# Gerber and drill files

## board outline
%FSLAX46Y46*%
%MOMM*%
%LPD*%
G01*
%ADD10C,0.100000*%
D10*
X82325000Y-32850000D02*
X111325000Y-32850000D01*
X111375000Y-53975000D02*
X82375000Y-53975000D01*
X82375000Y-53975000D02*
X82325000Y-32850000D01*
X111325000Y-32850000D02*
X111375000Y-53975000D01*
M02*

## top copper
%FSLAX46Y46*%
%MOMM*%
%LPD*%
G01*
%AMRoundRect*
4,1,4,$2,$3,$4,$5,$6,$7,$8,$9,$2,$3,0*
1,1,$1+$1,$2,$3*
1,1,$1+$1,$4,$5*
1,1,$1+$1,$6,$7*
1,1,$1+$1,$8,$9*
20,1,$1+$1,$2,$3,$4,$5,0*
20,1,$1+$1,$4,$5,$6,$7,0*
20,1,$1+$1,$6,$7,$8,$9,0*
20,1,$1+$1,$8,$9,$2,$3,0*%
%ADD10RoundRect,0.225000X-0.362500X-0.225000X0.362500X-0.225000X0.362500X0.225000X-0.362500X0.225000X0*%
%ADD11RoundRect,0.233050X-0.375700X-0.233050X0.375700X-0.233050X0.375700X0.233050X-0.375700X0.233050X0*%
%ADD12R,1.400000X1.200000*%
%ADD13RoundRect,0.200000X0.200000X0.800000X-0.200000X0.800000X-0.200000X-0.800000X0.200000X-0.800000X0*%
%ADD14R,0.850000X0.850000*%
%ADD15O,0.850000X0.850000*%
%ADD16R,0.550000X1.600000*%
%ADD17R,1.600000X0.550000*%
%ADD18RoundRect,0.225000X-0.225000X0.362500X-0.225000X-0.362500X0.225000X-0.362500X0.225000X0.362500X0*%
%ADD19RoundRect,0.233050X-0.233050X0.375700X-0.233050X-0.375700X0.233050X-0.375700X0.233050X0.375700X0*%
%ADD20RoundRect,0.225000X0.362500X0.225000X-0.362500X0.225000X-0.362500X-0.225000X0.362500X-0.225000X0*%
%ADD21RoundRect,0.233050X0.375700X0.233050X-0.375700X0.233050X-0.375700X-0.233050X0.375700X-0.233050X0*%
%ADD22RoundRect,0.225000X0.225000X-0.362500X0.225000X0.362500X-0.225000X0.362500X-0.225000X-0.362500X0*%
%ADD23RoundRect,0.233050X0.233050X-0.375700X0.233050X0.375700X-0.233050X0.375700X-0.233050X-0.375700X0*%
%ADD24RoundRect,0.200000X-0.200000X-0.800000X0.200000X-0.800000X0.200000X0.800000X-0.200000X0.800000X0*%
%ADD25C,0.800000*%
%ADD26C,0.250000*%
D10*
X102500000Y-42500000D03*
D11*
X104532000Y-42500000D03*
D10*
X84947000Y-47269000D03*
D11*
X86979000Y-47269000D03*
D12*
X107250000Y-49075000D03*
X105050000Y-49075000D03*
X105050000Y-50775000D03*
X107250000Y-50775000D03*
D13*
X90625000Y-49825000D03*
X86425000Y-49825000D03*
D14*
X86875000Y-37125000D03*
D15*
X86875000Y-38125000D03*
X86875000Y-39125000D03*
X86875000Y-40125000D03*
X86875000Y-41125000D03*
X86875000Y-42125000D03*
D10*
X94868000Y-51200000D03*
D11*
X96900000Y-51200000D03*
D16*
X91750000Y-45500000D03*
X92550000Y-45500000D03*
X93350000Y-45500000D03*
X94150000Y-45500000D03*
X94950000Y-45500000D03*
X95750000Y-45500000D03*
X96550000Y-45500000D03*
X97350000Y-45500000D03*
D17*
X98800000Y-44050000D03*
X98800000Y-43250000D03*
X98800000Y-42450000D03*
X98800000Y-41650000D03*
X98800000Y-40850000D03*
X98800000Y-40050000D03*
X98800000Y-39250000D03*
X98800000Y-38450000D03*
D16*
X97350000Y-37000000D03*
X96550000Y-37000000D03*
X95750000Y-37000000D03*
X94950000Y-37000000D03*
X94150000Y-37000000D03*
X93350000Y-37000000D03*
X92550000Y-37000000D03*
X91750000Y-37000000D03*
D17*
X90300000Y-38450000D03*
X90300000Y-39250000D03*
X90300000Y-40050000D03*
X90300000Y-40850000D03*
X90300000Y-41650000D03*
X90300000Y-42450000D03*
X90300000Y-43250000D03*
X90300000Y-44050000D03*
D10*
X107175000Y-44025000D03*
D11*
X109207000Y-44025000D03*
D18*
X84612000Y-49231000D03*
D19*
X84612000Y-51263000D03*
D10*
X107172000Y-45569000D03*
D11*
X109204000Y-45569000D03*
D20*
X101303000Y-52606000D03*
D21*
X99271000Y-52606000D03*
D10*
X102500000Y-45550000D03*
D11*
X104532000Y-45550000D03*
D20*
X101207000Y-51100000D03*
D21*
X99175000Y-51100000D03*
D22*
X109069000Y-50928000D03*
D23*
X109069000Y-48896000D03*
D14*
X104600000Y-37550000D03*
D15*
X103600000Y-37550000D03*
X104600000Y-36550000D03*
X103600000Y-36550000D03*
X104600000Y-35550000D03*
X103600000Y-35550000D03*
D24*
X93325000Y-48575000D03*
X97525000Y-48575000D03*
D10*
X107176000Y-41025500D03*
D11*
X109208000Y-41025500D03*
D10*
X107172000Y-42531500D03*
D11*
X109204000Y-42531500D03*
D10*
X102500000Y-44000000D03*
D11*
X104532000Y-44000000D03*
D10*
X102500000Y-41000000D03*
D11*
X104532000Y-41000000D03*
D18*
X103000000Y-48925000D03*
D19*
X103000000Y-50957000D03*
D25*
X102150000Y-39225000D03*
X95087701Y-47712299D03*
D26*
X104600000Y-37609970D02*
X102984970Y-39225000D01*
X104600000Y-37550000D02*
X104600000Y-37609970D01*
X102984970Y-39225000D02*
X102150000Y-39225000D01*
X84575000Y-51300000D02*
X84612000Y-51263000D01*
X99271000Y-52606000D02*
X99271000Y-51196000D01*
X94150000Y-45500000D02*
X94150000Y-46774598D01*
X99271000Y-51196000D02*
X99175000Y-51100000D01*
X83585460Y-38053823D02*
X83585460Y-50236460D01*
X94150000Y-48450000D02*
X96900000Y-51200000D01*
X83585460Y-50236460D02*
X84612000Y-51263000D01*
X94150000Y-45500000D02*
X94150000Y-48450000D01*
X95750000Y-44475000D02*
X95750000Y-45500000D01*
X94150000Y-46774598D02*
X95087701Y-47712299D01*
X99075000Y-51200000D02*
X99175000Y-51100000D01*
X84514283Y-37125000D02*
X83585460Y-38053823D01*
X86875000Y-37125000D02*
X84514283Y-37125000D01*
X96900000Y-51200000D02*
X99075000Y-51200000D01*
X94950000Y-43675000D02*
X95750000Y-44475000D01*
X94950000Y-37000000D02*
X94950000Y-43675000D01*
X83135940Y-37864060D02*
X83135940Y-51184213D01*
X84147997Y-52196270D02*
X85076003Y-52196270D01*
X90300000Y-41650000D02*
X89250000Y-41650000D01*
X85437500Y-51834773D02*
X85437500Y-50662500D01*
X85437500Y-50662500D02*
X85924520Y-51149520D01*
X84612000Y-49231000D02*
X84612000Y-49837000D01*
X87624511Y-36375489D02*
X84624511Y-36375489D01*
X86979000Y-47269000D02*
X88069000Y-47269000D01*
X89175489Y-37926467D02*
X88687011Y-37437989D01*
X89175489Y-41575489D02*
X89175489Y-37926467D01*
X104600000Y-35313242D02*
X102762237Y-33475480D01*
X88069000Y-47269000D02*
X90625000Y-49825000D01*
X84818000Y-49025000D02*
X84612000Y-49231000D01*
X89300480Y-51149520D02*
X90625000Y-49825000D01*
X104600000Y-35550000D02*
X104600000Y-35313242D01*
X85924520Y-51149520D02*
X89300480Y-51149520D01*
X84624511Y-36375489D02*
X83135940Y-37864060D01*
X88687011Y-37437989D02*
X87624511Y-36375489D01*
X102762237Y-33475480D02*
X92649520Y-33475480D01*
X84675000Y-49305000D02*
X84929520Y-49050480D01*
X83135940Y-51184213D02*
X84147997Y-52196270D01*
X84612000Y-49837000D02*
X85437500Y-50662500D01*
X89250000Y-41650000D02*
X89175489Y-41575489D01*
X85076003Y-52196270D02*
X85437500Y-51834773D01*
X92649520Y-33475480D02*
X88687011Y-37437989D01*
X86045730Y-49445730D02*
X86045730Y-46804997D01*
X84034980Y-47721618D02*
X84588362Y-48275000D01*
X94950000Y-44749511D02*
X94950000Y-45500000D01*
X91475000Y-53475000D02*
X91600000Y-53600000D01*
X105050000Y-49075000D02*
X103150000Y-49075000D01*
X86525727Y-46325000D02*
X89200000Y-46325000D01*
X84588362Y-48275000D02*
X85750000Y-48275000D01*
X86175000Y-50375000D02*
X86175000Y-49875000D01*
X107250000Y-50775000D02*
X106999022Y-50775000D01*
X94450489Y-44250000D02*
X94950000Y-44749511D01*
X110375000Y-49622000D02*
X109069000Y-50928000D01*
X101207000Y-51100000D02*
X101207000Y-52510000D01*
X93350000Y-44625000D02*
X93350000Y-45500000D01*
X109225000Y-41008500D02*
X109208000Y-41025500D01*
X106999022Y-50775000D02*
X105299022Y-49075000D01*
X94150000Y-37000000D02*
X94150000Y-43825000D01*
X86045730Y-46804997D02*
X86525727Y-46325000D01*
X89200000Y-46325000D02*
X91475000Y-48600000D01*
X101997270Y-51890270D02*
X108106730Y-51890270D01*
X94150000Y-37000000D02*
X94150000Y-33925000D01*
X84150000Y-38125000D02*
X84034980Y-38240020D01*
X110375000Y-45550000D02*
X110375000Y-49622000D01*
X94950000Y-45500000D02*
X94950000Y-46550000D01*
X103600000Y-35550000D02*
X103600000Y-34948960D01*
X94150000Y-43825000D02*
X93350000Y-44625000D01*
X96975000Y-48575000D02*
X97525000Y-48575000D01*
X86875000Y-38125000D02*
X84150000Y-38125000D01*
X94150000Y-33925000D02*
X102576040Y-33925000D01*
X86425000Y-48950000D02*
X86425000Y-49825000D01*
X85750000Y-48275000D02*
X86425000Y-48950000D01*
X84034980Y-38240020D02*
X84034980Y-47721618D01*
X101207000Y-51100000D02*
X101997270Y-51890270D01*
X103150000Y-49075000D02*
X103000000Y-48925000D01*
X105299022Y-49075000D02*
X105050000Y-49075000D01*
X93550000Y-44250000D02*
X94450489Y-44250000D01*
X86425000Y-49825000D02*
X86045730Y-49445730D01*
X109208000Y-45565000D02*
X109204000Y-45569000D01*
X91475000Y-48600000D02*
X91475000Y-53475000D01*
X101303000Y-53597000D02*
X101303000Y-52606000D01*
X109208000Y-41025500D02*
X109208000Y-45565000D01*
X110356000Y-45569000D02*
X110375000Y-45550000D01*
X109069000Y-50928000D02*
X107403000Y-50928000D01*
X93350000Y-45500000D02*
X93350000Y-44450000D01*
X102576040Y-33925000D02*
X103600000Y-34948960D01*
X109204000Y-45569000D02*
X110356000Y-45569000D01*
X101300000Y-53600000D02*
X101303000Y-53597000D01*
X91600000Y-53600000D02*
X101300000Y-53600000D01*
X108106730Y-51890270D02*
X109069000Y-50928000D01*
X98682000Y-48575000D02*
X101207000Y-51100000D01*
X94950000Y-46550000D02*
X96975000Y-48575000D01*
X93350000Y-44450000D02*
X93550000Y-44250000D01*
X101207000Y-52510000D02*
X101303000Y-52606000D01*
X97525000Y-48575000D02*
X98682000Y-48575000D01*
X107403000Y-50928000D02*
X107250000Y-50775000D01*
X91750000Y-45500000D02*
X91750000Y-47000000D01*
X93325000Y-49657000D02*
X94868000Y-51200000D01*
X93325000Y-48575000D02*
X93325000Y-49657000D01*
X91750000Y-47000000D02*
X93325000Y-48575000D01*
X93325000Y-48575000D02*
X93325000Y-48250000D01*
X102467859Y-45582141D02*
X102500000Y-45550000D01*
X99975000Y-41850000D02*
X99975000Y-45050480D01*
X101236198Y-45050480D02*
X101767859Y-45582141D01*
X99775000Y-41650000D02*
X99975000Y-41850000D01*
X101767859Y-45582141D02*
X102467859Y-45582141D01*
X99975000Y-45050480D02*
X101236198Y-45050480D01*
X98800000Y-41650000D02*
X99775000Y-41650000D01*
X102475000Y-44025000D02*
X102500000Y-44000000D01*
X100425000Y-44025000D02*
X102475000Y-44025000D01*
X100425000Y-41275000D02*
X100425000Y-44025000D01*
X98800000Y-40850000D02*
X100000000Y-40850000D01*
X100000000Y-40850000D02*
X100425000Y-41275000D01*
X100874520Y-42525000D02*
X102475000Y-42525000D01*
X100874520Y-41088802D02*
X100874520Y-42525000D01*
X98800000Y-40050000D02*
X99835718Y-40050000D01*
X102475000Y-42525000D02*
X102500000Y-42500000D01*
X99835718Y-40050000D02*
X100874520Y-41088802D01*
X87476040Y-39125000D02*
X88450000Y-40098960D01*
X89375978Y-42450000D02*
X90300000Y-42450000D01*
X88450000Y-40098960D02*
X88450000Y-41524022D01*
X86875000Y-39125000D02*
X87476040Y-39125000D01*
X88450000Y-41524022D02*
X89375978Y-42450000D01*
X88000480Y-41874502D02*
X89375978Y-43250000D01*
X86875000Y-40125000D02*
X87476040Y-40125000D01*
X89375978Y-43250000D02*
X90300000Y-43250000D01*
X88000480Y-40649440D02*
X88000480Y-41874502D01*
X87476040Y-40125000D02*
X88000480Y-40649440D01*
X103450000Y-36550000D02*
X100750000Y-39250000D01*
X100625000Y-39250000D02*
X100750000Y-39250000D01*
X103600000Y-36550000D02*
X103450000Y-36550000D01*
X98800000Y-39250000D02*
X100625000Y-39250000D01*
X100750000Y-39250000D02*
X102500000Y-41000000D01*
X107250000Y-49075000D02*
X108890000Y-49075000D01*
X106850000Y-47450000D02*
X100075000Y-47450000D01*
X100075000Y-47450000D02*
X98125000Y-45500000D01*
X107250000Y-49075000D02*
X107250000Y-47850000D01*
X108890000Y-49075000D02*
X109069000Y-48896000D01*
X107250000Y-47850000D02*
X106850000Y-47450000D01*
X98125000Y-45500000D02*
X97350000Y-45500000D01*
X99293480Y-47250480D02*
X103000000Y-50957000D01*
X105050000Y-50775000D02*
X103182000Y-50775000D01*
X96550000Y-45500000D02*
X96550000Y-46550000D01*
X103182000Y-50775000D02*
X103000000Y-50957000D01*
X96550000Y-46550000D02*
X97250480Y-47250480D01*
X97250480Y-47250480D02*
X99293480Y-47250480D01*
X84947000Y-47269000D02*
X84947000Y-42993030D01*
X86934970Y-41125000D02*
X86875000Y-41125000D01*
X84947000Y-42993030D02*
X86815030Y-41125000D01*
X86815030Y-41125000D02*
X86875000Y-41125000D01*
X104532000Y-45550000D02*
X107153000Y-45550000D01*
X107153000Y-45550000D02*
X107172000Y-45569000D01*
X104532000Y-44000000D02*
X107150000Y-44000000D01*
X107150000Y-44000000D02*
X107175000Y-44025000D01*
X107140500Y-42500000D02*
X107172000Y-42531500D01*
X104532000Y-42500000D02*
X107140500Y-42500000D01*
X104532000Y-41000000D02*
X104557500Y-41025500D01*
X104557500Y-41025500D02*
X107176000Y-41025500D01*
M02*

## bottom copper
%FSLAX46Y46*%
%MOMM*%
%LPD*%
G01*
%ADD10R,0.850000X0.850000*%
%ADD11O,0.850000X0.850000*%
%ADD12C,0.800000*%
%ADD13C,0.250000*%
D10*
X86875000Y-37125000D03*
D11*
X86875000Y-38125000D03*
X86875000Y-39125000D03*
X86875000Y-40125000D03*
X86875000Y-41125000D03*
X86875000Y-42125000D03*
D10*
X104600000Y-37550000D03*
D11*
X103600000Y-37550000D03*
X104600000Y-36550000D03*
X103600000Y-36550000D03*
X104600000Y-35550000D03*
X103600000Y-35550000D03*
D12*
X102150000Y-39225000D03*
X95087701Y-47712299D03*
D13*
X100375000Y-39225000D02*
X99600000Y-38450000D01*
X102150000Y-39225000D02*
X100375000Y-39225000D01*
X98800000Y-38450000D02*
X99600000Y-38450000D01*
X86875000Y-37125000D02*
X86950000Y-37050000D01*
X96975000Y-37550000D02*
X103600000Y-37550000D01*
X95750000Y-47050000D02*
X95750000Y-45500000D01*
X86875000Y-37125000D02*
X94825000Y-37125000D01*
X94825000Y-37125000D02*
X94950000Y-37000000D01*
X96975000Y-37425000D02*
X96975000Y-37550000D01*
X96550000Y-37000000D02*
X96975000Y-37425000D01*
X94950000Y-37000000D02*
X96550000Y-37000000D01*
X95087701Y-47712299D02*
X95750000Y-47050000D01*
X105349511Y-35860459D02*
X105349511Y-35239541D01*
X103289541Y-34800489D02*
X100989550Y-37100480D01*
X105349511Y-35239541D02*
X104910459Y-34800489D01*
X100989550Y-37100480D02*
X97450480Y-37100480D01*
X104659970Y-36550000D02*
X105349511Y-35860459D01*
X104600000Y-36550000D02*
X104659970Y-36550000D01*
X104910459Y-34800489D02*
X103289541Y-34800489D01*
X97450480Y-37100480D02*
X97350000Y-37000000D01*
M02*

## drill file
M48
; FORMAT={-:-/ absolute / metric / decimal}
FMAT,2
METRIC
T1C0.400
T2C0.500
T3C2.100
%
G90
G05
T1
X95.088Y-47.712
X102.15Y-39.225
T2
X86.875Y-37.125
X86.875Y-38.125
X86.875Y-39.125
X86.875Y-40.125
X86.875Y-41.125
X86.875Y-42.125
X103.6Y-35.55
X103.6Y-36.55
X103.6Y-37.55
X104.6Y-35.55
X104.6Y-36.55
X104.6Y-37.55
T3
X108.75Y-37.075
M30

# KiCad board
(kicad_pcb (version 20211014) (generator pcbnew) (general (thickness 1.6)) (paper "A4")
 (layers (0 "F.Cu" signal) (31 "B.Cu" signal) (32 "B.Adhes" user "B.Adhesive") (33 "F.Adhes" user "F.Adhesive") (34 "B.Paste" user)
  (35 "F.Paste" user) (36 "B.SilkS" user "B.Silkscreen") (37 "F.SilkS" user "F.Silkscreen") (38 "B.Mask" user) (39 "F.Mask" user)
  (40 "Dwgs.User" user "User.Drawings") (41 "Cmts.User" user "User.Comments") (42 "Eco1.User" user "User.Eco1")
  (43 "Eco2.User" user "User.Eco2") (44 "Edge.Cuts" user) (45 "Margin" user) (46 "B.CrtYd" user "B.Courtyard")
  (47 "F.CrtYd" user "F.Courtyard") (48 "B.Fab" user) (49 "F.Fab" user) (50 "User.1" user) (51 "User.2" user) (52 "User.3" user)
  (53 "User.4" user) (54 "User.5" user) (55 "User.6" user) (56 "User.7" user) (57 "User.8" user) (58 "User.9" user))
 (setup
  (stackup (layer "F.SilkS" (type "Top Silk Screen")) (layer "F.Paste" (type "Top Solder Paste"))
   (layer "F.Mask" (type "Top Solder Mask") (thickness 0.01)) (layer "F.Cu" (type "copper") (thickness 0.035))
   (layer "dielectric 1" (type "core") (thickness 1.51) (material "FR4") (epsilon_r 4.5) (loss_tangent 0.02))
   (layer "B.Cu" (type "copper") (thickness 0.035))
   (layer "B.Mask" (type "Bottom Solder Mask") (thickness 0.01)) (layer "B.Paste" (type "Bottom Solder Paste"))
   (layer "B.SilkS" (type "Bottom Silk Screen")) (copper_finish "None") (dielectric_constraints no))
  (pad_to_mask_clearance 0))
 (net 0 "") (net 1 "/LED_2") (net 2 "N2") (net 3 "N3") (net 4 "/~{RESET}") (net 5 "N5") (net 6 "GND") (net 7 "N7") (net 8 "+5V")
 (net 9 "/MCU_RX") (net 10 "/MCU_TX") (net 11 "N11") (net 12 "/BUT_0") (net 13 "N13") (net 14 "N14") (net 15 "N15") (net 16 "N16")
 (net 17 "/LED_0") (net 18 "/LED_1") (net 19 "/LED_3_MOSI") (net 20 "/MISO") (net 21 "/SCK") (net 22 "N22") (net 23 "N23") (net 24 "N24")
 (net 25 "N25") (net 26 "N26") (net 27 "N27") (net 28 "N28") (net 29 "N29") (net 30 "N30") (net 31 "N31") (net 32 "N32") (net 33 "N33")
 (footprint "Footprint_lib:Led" (layer "F.Cu") (at 103.478 42.481)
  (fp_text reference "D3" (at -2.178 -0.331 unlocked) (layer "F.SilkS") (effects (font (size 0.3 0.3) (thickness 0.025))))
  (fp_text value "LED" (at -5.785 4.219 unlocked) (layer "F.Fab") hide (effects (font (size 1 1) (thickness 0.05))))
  (pad "1" smd roundrect (at -0.978 0.019) (size 1.175 0.9) (layers "F.Cu" "F.Paste" "F.Mask") (roundrect_rratio 0.25) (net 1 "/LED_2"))
  (pad "2" smd roundrect (at 1.054 0.019) (size 1.2175 0.9322) (layers "F.Cu" "F.Paste" "F.Mask") (roundrect_rratio 0.25) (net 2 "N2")))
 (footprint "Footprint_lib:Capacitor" (layer "F.Cu") (at 85.95 47.25)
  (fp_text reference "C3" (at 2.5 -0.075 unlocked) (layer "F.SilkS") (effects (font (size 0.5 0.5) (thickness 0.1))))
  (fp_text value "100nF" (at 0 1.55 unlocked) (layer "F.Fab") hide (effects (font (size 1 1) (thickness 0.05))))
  (pad "1" smd roundrect (at -1.003 0.019) (size 1.175 0.9) (layers "F.Cu" "F.Paste" "F.Mask") (roundrect_rratio 0.25) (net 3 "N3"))
  (pad "2" smd roundrect (at 1.029 0.019) (size 1.2175 0.9322) (layers "F.Cu" "F.Paste" "F.Mask") (roundrect_rratio 0.25)
   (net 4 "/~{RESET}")))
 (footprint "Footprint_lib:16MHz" (layer "F.Cu") (at 106.15 49.875 180)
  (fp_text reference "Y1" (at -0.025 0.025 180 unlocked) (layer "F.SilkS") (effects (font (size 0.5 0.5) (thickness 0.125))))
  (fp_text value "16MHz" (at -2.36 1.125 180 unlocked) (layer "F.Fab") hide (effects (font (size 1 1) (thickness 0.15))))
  (pad "1" smd rect (at -1.1 0.8 180) (size 1.4 1.2) (layers "F.Cu" "F.Paste" "F.Mask") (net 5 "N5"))
  (pad "2" smd rect (at 1.1 0.8 180) (size 1.4 1.2) (layers "F.Cu" "F.Paste" "F.Mask") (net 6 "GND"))
  (pad "3" smd rect (at 1.1 -0.9 180) (size 1.4 1.2) (layers "F.Cu" "F.Paste" "F.Mask") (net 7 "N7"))
  (pad "4" smd rect (at -1.1 -0.9 180) (size 1.4 1.2) (layers "F.Cu" "F.Paste" "F.Mask") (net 6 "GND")))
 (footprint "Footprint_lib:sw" (layer "F.Cu") (at 88.525 49.895 180)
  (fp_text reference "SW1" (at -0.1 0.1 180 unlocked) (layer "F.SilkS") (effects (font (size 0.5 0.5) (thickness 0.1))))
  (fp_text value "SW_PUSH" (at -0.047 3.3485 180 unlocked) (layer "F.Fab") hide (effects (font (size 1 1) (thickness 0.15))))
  (pad "1" smd roundrect (at -2.1 0.07 180) (size 0.8 2) (layers "F.Cu" "F.Paste" "F.Mask") (roundrect_rratio 0.25) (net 4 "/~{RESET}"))
  (pad "2" smd roundrect (at 2.1 0.07 180) (size 0.8 2) (layers "F.Cu" "F.Paste" "F.Mask") (roundrect_rratio 0.25) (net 6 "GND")))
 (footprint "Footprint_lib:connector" (layer "F.Cu") (at 86.875 39.625)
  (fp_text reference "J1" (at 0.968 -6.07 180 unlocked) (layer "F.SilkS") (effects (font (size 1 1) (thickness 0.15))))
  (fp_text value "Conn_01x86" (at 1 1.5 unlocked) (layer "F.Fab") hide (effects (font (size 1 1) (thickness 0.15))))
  (pad "1" thru_hole rect (at 0 -2.5) (size 0.85 0.85) (drill 0.5) (layers *.Cu *.Mask) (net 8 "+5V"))
  (pad "2" thru_hole oval (at 0 -1.5) (size 0.85 0.85) (drill 0.5) (layers *.Cu *.Mask) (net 6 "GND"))
  (pad "3" thru_hole oval (at 0 -0.5) (size 0.85 0.85) (drill 0.5) (layers *.Cu *.Mask) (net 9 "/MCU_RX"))
  (pad "4" thru_hole oval (at 0 0.5) (size 0.85 0.85) (drill 0.5) (layers *.Cu *.Mask) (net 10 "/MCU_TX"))
  (pad "5" thru_hole oval (at 0 1.5) (size 0.85 0.85) (drill 0.5) (layers *.Cu *.Mask) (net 3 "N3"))
  (pad "6" thru_hole oval (at 0 2.5) (size 0.85 0.85) (drill 0.5) (layers *.Cu *.Mask) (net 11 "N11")))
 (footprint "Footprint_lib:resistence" (layer "F.Cu") (at 95.921 51.1685)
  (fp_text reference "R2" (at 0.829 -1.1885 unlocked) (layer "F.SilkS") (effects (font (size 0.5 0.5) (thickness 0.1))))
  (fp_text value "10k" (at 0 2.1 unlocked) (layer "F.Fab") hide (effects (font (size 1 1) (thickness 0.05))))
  (pad "1" smd roundrect (at -1.053 0.0315) (size 1.175 0.9) (layers "F.Cu" "F.Paste" "F.Mask") (roundrect_rratio 0.25) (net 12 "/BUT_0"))
  (pad "2" smd roundrect (at 0.979 0.0315) (size 1.2175 0.9322) (layers "F.Cu" "F.Paste" "F.Mask") (roundrect_rratio 0.25) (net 8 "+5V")))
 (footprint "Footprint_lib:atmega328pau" (layer "F.Cu") (at 94.55 41.25 90)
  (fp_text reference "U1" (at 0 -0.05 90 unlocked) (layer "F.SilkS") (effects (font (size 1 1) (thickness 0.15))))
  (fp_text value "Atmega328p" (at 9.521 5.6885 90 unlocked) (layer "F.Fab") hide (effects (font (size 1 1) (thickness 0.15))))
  (pad "1" smd rect (at -4.25 -2.8 90) (size 1.6 0.55) (layers "F.Cu" "F.Paste" "F.Mask") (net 12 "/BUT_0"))
  (pad "2" smd rect (at -4.25 -2 90) (size 1.6 0.55) (layers "F.Cu" "F.Paste" "F.Mask") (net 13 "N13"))
  (pad "3" smd rect (at -4.25 -1.2 90) (size 1.6 0.55) (layers "F.Cu" "F.Paste" "F.Mask") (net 6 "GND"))
  (pad "4" smd rect (at -4.25 -0.4 90) (size 1.6 0.55) (layers "F.Cu" "F.Paste" "F.Mask") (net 8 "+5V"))
  (pad "5" smd rect (at -4.25 0.4 90) (size 1.6 0.55) (layers "F.Cu" "F.Paste" "F.Mask") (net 6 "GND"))
  (pad "6" smd rect (at -4.25 1.2 90) (size 1.6 0.55) (layers "F.Cu" "F.Paste" "F.Mask") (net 8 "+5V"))
  (pad "7" smd rect (at -4.25 2 90) (size 1.6 0.55) (layers "F.Cu" "F.Paste" "F.Mask") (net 7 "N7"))
  (pad "8" smd rect (at -4.25 2.8 90) (size 1.6 0.55) (layers "F.Cu" "F.Paste" "F.Mask") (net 5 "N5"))
  (pad "9" smd rect (at -2.8 4.25 180) (size 1.6 0.55) (layers "F.Cu" "F.Paste" "F.Mask") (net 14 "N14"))
  (pad "10" smd rect (at -2 4.25 180) (size 1.6 0.55) (layers "F.Cu" "F.Paste" "F.Mask") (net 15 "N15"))
  (pad "11" smd rect (at -1.2 4.25 180) (size 1.6 0.55) (layers "F.Cu" "F.Paste" "F.Mask") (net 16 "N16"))
  (pad "12" smd rect (at -0.4 4.25 180) (size 1.6 0.55) (layers "F.Cu" "F.Paste" "F.Mask") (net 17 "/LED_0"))
  (pad "13" smd rect (at 0.4 4.25 180) (size 1.6 0.55) (layers "F.Cu" "F.Paste" "F.Mask") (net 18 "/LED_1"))
  (pad "14" smd rect (at 1.2 4.25 180) (size 1.6 0.55) (layers "F.Cu" "F.Paste" "F.Mask") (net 1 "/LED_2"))
  (pad "15" smd rect (at 2 4.25 180) (size 1.6 0.55) (layers "F.Cu" "F.Paste" "F.Mask") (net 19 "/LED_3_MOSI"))
  (pad "16" smd rect (at 2.8 4.25 180) (size 1.6 0.55) (layers "F.Cu" "F.Paste" "F.Mask") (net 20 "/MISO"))
  (pad "17" smd rect (at 4.25 2.8 90) (size 1.6 0.55) (layers "F.Cu" "F.Paste" "F.Mask") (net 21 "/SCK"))
  (pad "18" smd rect (at 4.25 2 90) (size 1.6 0.55) (layers "F.Cu" "F.Paste" "F.Mask") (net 8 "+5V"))
  (pad "19" smd rect (at 4.25 1.2 90) (size 1.6 0.55) (layers "F.Cu" "F.Paste" "F.Mask") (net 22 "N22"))
  (pad "20" smd rect (at 4.25 0.4 90) (size 1.6 0.55) (layers "F.Cu" "F.Paste" "F.Mask") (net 8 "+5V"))
  (pad "21" smd rect (at 4.25 -0.4 90) (size 1.6 0.55) (layers "F.Cu" "F.Paste" "F.Mask") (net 6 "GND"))
  (pad "22" smd rect (at 4.25 -1.2 90) (size 1.6 0.55) (layers "F.Cu" "F.Paste" "F.Mask") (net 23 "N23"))
  (pad "23" smd rect (at 4.25 -2 90) (size 1.6 0.55) (layers "F.Cu" "F.Paste" "F.Mask") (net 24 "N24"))
  (pad "24" smd rect (at 4.25 -2.8 90) (size 1.6 0.55) (layers "F.Cu" "F.Paste" "F.Mask") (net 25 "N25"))
  (pad "25" smd rect (at 2.8 -4.25 180) (size 1.6 0.55) (layers "F.Cu" "F.Paste" "F.Mask") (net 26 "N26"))
  (pad "26" smd rect (at 2 -4.25 180) (size 1.6 0.55) (layers "F.Cu" "F.Paste" "F.Mask") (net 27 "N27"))
  (pad "27" smd rect (at 1.2 -4.25 180) (size 1.6 0.55) (layers "F.Cu" "F.Paste" "F.Mask") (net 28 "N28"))
  (pad "28" smd rect (at 0.4 -4.25 180) (size 1.6 0.55) (layers "F.Cu" "F.Paste" "F.Mask") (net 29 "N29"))
  (pad "29" smd rect (at -0.4 -4.25 180) (size 1.6 0.55) (layers "F.Cu" "F.Paste" "F.Mask") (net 4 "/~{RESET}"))
  (pad "30" smd rect (at -1.2 -4.25 180) (size 1.6 0.55) (layers "F.Cu" "F.Paste" "F.Mask") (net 9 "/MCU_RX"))
  (pad "31" smd rect (at -2 -4.25 180) (size 1.6 0.55) (layers "F.Cu" "F.Paste" "F.Mask") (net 10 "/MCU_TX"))
  (pad "32" smd rect (at -2.8 -4.25 180) (size 1.6 0.55) (layers "F.Cu" "F.Paste" "F.Mask") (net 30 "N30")))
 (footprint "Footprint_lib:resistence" (layer "F.Cu") (at 108.228 43.9935)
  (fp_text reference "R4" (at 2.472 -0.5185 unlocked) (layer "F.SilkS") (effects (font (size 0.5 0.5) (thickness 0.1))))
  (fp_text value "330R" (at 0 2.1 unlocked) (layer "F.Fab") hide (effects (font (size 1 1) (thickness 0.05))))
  (pad "1" smd roundrect (at -1.053 0.0315) (size 1.175 0.9) (layers "F.Cu" "F.Paste" "F.Mask") (roundrect_rratio 0.25) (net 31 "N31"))
  (pad "2" smd roundrect (at 0.979 0.0315) (size 1.2175 0.9322) (layers "F.Cu" "F.Paste" "F.Mask") (roundrect_rratio 0.25) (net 6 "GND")))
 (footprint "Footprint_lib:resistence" (layer "F.Cu") (at 84.6435 50.284 -90)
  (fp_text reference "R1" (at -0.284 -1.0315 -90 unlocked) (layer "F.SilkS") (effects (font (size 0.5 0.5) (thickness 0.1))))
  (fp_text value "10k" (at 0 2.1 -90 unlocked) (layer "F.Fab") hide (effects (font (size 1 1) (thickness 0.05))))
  (pad "1" smd roundrect (at -1.053 0.0315 270) (size 1.175 0.9) (layers "F.Cu" "F.Paste" "F.Mask") (roundrect_rratio 0.25)
   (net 4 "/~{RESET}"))
  (pad "2" smd roundrect (at 0.979 0.0315 270) (size 1.2175 0.9322) (layers "F.Cu" "F.Paste" "F.Mask") (roundrect_rratio 0.25) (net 8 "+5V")))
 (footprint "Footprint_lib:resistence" (layer "F.Cu") (at 108.225 45.5375)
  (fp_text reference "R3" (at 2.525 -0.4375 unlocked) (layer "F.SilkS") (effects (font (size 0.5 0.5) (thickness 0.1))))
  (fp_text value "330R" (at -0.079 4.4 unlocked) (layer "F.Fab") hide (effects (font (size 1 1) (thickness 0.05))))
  (pad "1" smd roundrect (at -1.053 0.0315) (size 1.175 0.9) (layers "F.Cu" "F.Paste" "F.Mask") (roundrect_rratio 0.25) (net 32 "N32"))
  (pad "2" smd roundrect (at 0.979 0.0315) (size 1.2175 0.9322) (layers "F.Cu" "F.Paste" "F.Mask") (roundrect_rratio 0.25) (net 6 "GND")))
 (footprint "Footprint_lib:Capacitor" (layer "F.Cu") (at 100.3 52.625 180)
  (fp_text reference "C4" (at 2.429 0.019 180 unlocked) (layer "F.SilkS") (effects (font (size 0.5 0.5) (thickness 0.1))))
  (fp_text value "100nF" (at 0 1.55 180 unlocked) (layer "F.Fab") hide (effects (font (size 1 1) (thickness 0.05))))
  (pad "1" smd roundrect (at -1.003 0.019 180) (size 1.175 0.9) (layers "F.Cu" "F.Paste" "F.Mask") (roundrect_rratio 0.25) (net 6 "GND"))
  (pad "2" smd roundrect (at 1.029 0.019 180) (size 1.2175 0.9322) (layers "F.Cu" "F.Paste" "F.Mask") (roundrect_rratio 0.25) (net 8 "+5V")))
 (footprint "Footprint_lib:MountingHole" (layer "F.Cu") (at 108.75 37.075)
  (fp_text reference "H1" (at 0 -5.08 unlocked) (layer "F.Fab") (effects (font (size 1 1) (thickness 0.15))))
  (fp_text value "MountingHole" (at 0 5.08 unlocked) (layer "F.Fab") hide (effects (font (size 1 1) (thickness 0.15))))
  (pad "" np_thru_hole circle (at 0 0) (size 2.1 2.1) (drill 2.1) (layers *.Cu *.Mask)))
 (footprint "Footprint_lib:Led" (layer "F.Cu") (at 103.478 45.531)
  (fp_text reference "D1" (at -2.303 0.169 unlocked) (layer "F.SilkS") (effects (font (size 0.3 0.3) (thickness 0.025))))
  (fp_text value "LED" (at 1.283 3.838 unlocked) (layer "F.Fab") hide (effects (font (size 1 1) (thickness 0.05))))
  (pad "1" smd roundrect (at -0.978 0.019) (size 1.175 0.9) (layers "F.Cu" "F.Paste" "F.Mask") (roundrect_rratio 0.25) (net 17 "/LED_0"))
  (pad "2" smd roundrect (at 1.054 0.019) (size 1.2175 0.9322) (layers "F.Cu" "F.Paste" "F.Mask") (roundrect_rratio 0.25) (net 32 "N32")))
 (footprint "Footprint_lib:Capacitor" (layer "F.Cu") (at 100.204 51.119 180)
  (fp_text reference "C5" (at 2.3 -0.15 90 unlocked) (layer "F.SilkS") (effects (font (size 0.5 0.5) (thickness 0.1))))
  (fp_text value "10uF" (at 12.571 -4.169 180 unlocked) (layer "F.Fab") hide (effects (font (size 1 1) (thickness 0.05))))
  (pad "1" smd roundrect (at -1.003 0.019 180) (size 1.175 0.9) (layers "F.Cu" "F.Paste" "F.Mask") (roundrect_rratio 0.25) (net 6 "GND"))
  (pad "2" smd roundrect (at 1.029 0.019 180) (size 1.2175 0.9322) (layers "F.Cu" "F.Paste" "F.Mask") (roundrect_rratio 0.25) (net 8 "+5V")))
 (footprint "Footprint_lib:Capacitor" (layer "F.Cu") (at 109.05 49.925 90)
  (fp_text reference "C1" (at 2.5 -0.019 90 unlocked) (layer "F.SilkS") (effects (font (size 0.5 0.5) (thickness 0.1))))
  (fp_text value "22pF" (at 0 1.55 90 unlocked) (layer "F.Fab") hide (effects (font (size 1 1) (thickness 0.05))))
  (pad "1" smd roundrect (at -1.003 0.019 90) (size 1.175 0.9) (layers "F.Cu" "F.Paste" "F.Mask") (roundrect_rratio 0.25) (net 6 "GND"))
  (pad "2" smd roundrect (at 1.029 0.019 90) (size 1.2175 0.9322) (layers "F.Cu" "F.Paste" "F.Mask") (roundrect_rratio 0.25) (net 5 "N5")))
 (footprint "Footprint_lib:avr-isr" (layer "F.Cu") (at 104.15 36.55 180)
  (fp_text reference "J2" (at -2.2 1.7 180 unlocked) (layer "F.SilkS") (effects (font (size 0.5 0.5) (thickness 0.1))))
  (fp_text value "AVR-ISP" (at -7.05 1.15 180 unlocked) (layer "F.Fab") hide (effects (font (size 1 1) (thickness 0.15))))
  (pad "1" thru_hole rect (at -0.45 -1 180) (size 0.85 0.85) (drill 0.5) (layers *.Cu *.Mask) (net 20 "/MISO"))
  (pad "2" thru_hole oval (at 0.55 -1 180) (size 0.85 0.85) (drill 0.5) (layers *.Cu *.Mask) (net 8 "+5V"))
  (pad "3" thru_hole oval (at -0.45 0 180) (size 0.85 0.85) (drill 0.5) (layers *.Cu *.Mask) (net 21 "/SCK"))
  (pad "4" thru_hole oval (at 0.55 0 180) (size 0.85 0.85) (drill 0.5) (layers *.Cu *.Mask) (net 19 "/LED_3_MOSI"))
  (pad "5" thru_hole oval (at -0.45 1 180) (size 0.85 0.85) (drill 0.5) (layers *.Cu *.Mask) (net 4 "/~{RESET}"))
  (pad "6" thru_hole oval (at 0.55 1 180) (size 0.85 0.85) (drill 0.5) (layers *.Cu *.Mask) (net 6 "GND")))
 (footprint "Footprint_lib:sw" (layer "F.Cu") (at 95.425 48.505)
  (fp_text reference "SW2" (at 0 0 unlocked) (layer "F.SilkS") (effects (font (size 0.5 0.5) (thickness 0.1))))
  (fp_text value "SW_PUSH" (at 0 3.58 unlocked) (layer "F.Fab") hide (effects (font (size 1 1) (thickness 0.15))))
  (pad "1" smd roundrect (at -2.1 0.07) (size 0.8 2) (layers "F.Cu" "F.Paste" "F.Mask") (roundrect_rratio 0.25) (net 12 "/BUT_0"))
  (pad "2" smd roundrect (at 2.1 0.07) (size 0.8 2) (layers "F.Cu" "F.Paste" "F.Mask") (roundrect_rratio 0.25) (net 6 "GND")))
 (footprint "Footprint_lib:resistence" (layer "F.Cu") (at 108.229 40.994)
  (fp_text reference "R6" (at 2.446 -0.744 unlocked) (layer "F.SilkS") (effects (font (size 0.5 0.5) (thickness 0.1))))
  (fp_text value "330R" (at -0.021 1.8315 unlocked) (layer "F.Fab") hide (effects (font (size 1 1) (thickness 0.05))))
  (pad "1" smd roundrect (at -1.053 0.0315) (size 1.175 0.9) (layers "F.Cu" "F.Paste" "F.Mask") (roundrect_rratio 0.25) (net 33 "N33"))
  (pad "2" smd roundrect (at 0.979 0.0315) (size 1.2175 0.9322) (layers "F.Cu" "F.Paste" "F.Mask") (roundrect_rratio 0.25) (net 6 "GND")))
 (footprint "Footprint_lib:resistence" (layer "F.Cu") (at 108.225 42.5)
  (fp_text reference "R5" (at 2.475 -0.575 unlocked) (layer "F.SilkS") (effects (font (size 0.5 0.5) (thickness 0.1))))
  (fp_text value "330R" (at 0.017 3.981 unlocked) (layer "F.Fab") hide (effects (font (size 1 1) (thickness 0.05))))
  (pad "1" smd roundrect (at -1.053 0.0315) (size 1.175 0.9) (layers "F.Cu" "F.Paste" "F.Mask") (roundrect_rratio 0.25) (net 2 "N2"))
  (pad "2" smd roundrect (at 0.979 0.0315) (size 1.2175 0.9322) (layers "F.Cu" "F.Paste" "F.Mask") (roundrect_rratio 0.25) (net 6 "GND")))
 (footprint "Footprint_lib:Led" (layer "F.Cu") (at 103.478 43.981)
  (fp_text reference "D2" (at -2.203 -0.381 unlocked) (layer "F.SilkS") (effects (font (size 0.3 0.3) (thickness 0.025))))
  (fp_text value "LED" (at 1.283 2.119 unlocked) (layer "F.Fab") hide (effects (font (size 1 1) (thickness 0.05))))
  (pad "1" smd roundrect (at -0.978 0.019) (size 1.175 0.9) (layers "F.Cu" "F.Paste" "F.Mask") (roundrect_rratio 0.25) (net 18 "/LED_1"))
  (pad "2" smd roundrect (at 1.054 0.019) (size 1.2175 0.9322) (layers "F.Cu" "F.Paste" "F.Mask") (roundrect_rratio 0.25) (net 31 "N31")))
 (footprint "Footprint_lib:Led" (layer "F.Cu") (at 103.478 40.981)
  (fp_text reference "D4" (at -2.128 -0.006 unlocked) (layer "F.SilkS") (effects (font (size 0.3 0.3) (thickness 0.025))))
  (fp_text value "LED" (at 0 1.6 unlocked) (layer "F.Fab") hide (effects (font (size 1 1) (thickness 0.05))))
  (pad "1" smd roundrect (at -0.978 0.019) (size 1.175 0.9) (layers "F.Cu" "F.Paste" "F.Mask") (roundrect_rratio 0.25)
   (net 19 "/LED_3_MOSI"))
  (pad "2" smd roundrect (at 1.054 0.019) (size 1.2175 0.9322) (layers "F.Cu" "F.Paste" "F.Mask") (roundrect_rratio 0.25) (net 33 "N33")))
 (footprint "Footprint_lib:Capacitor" (layer "F.Cu") (at 103.019 49.928 -90)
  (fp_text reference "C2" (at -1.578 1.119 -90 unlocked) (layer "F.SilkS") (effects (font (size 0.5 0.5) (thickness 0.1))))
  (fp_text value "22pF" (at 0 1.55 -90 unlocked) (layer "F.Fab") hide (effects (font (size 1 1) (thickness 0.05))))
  (pad "1" smd roundrect (at -1.003 0.019 270) (size 1.175 0.9) (layers "F.Cu" "F.Paste" "F.Mask") (roundrect_rratio 0.25) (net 6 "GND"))
  (pad "2" smd roundrect (at 1.029 0.019 270) (size 1.2175 0.9322) (layers "F.Cu" "F.Paste" "F.Mask") (roundrect_rratio 0.25) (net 7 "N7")))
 (gr_line (start 82.325 32.85) (end 111.325 32.85) (layer "Edge.Cuts") (width 0.1))
 (gr_line (start 111.375 53.975) (end 82.375 53.975) (layer "Edge.Cuts") (width 0.1))
 (gr_line (start 82.375 53.975) (end 82.325 32.85) (layer "Edge.Cuts") (width 0.1))
 (gr_line (start 111.325 32.85) (end 111.375 53.975) (layer "Edge.Cuts") (width 0.1))
 (segment (start 104.6 37.60997) (end 102.98497 39.225) (width 0.25) (layer "F.Cu") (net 20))
 (segment (start 104.6 37.55) (end 104.6 37.60997) (width 0.25) (layer "F.Cu") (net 20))
 (segment (start 102.98497 39.225) (end 102.15 39.225) (width 0.25) (layer "F.Cu") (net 20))
 (via (at 102.15 39.225) (size 0.8) (drill 0.4) (layers "F.Cu" "B.Cu") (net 20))
 (segment (start 100.375 39.225) (end 99.6 38.45) (width 0.25) (layer "B.Cu") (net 20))
 (segment (start 102.15 39.225) (end 100.375 39.225) (width 0.25) (layer "B.Cu") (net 20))
 (segment (start 98.8 38.45) (end 99.6 38.45) (width 0.25) (layer "B.Cu") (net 20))
 (segment (start 84.575 51.3) (end 84.612 51.263) (width 0.25) (layer "F.Cu") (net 8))
 (segment (start 99.271 52.606) (end 99.271 51.196) (width 0.25) (layer "F.Cu") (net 8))
 (segment (start 94.15 45.5) (end 94.15 46.774598) (width 0.25) (layer "F.Cu") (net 8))
 (segment (start 99.271 51.196) (end 99.175 51.1) (width 0.25) (layer "F.Cu") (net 8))
 (segment (start 83.58546 38.053823) (end 83.58546 50.23646) (width 0.25) (layer "F.Cu") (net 8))
 (segment (start 94.15 48.45) (end 96.9 51.2) (width 0.25) (layer "F.Cu") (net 8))
 (segment (start 83.58546 50.23646) (end 84.612 51.263) (width 0.25) (layer "F.Cu") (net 8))
 (segment (start 94.15 45.5) (end 94.15 48.45) (width 0.25) (layer "F.Cu") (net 8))
 (segment (start 95.75 44.475) (end 95.75 45.5) (width 0.25) (layer "F.Cu") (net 8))
 (segment (start 94.15 46.774598) (end 95.087701 47.712299) (width 0.25) (layer "F.Cu") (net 8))
 (segment (start 99.075 51.2) (end 99.175 51.1) (width 0.25) (layer "F.Cu") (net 8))
 (segment (start 84.514283 37.125) (end 83.58546 38.053823) (width 0.25) (layer "F.Cu") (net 8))
 (segment (start 86.875 37.125) (end 84.514283 37.125) (width 0.25) (layer "F.Cu") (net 8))
 (segment (start 96.9 51.2) (end 99.075 51.2) (width 0.25) (layer "F.Cu") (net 8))
 (segment (start 94.95 43.675) (end 95.75 44.475) (width 0.25) (layer "F.Cu") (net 8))
 (segment (start 94.95 37) (end 94.95 43.675) (width 0.25) (layer "F.Cu") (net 8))
 (via (at 95.087701 47.712299) (size 0.8) (drill 0.4) (layers "F.Cu" "B.Cu") (remove_unused_layers) (keep_end_layers) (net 8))
 (segment (start 86.875 37.125) (end 86.95 37.05) (width 0.25) (layer "B.Cu") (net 8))
 (segment (start 96.975 37.55) (end 103.6 37.55) (width 0.25) (layer "B.Cu") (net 8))
 (segment (start 95.75 47.05) (end 95.75 45.5) (width 0.25) (layer "B.Cu") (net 8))
 (segment (start 86.875 37.125) (end 94.825 37.125) (width 0.25) (layer "B.Cu") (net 8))
 (segment (start 94.825 37.125) (end 94.95 37) (width 0.25) (layer "B.Cu") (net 8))
 (segment (start 96.975 37.425) (end 96.975 37.55) (width 0.25) (layer "B.Cu") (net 8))
 (segment (start 96.55 37) (end 96.975 37.425) (width 0.25) (layer "B.Cu") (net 8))
 (segment (start 94.95 37) (end 96.55 37) (width 0.25) (layer "B.Cu") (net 8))
 (segment (start 95.087701 47.712299) (end 95.75 47.05) (width 0.25) (layer "B.Cu") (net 8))
 (segment (start 105.349511 35.860459) (end 105.349511 35.239541) (width 0.25) (layer "B.Cu") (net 21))
 (segment (start 103.289541 34.800489) (end 100.98955 37.10048) (width 0.25) (layer "B.Cu") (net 21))
 (segment (start 105.349511 35.239541) (end 104.910459 34.800489) (width 0.25) (layer "B.Cu") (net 21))
 (segment (start 100.98955 37.10048) (end 97.45048 37.10048) (width 0.25) (layer "B.Cu") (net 21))
 (segment (start 104.65997 36.55) (end 105.349511 35.860459) (width 0.25) (layer "B.Cu") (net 21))
 (segment (start 104.6 36.55) (end 104.65997 36.55) (width 0.25) (layer "B.Cu") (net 21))
 (segment (start 104.910459 34.800489) (end 103.289541 34.800489) (width 0.25) (layer "B.Cu") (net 21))
 (segment (start 97.45048 37.10048) (end 97.35 37) (width 0.25) (layer "B.Cu") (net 21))
 (segment (start 83.13594 37.86406) (end 83.13594 51.184213) (width 0.25) (layer "F.Cu") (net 4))
 (segment (start 84.147997 52.19627) (end 85.076003 52.19627) (width 0.25) (layer "F.Cu") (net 4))
 (segment (start 90.3 41.65) (end 89.25 41.65) (width 0.25) (layer "F.Cu") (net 4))
 (segment (start 85.4375 51.834773) (end 85.4375 50.6625) (width 0.25) (layer "F.Cu") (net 4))
 (segment (start 85.4375 50.6625) (end 85.92452 51.14952) (width 0.25) (layer "F.Cu") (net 4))
 (segment (start 84.612 49.231) (end 84.612 49.837) (width 0.25) (layer "F.Cu") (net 4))
 (segment (start 87.624511 36.375489) (end 84.624511 36.375489) (width 0.25) (layer "F.Cu") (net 4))
 (segment (start 86.979 47.269) (end 88.069 47.269) (width 0.25) (layer "F.Cu") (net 4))
 (segment (start 89.175489 37.926467) (end 88.687011 37.437989) (width 0.25) (layer "F.Cu") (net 4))
 (segment (start 89.175489 41.575489) (end 89.175489 37.926467) (width 0.25) (layer "F.Cu") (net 4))
 (segment (start 104.6 35.313242) (end 102.762237 33.47548) (width 0.25) (layer "F.Cu") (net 4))
 (segment (start 88.069 47.269) (end 90.625 49.825) (width 0.25) (layer "F.Cu") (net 4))
 (segment (start 84.818 49.025) (end 84.612 49.231) (width 0.25) (layer "F.Cu") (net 4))
 (segment (start 89.30048 51.14952) (end 90.625 49.825) (width 0.25) (layer "F.Cu") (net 4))
 (segment (start 104.6 35.55) (end 104.6 35.313242) (width 0.25) (layer "F.Cu") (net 4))
 (segment (start 85.92452 51.14952) (end 89.30048 51.14952) (width 0.25) (layer "F.Cu") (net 4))
 (segment (start 84.624511 36.375489) (end 83.13594 37.86406) (width 0.25) (layer "F.Cu") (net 4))
 (segment (start 88.687011 37.437989) (end 87.624511 36.375489) (width 0.25) (layer "F.Cu") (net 4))
 (segment (start 102.762237 33.47548) (end 92.64952 33.47548) (width 0.25) (layer "F.Cu") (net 4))
 (segment (start 84.675 49.305) (end 84.92952 49.05048) (width 0.25) (layer "F.Cu") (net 4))
 (segment (start 83.13594 51.184213) (end 84.147997 52.19627) (width 0.25) (layer "F.Cu") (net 4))
 (segment (start 84.612 49.837) (end 85.4375 50.6625) (width 0.25) (layer "F.Cu") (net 4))
 (segment (start 89.25 41.65) (end 89.175489 41.575489) (width 0.25) (layer "F.Cu") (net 4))
 (segment (start 85.076003 52.19627) (end 85.4375 51.834773) (width 0.25) (layer "F.Cu") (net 4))
 (segment (start 92.64952 33.47548) (end 88.687011 37.437989) (width 0.25) (layer "F.Cu") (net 4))
 (segment (start 86.04573 49.44573) (end 86.04573 46.804997) (width 0.25) (layer "F.Cu") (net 6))
 (segment (start 84.03498 47.721618) (end 84.588362 48.275) (width 0.25) (layer "F.Cu") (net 6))
 (segment (start 94.95 44.749511) (end 94.95 45.5) (width 0.25) (layer "F.Cu") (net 6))
 (segment (start 91.475 53.475) (end 91.6 53.6) (width 0.25) (layer "F.Cu") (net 6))
 (segment (start 105.05 49.075) (end 103.15 49.075) (width 0.25) (layer "F.Cu") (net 6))
 (segment (start 86.525727 46.325) (end 89.2 46.325) (width 0.25) (layer "F.Cu") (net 6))
 (segment (start 84.588362 48.275) (end 85.75 48.275) (width 0.25) (layer "F.Cu") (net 6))
 (segment (start 86.175 50.375) (end 86.175 49.875) (width 0.25) (layer "F.Cu") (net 6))
 (segment (start 107.25 50.775) (end 106.999022 50.775) (width 0.25) (layer "F.Cu") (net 6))
 (segment (start 94.450489 44.25) (end 94.95 44.749511) (width 0.25) (layer "F.Cu") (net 6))
 (segment (start 110.375 49.622) (end 109.069 50.928) (width 0.25) (layer "F.Cu") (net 6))
 (segment (start 101.207 51.1) (end 101.207 52.51) (width 0.25) (layer "F.Cu") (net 6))
 (segment (start 93.35 44.625) (end 93.35 45.5) (width 0.25) (layer "F.Cu") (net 6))
 (segment (start 109.225 41.0085) (end 109.208 41.0255) (width 0.25) (layer "F.Cu") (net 6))
 (segment (start 106.999022 50.775) (end 105.299022 49.075) (width 0.25) (layer "F.Cu") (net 6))
 (segment (start 94.15 37) (end 94.15 43.825) (width 0.25) (layer "F.Cu") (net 6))
 (segment (start 86.04573 46.804997) (end 86.525727 46.325) (width 0.25) (layer "F.Cu") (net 6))
 (segment (start 89.2 46.325) (end 91.475 48.6) (width 0.25) (layer "F.Cu") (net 6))
 (segment (start 101.99727 51.89027) (end 108.10673 51.89027) (width 0.25) (layer "F.Cu") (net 6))
 (segment (start 94.15 37) (end 94.15 33.925) (width 0.25) (layer "F.Cu") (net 6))
 (segment (start 84.15 38.125) (end 84.03498 38.24002) (width 0.25) (layer "F.Cu") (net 6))
 (segment (start 110.375 45.55) (end 110.375 49.622) (width 0.25) (layer "F.Cu") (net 6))
 (segment (start 94.95 45.5) (end 94.95 46.55) (width 0.25) (layer "F.Cu") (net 6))
 (segment (start 103.6 35.55) (end 103.6 34.94896) (width 0.25) (layer "F.Cu") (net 6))
 (segment (start 94.15 43.825) (end 93.35 44.625) (width 0.25) (layer "F.Cu") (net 6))
 (segment (start 96.975 48.575) (end 97.525 48.575) (width 0.25) (layer "F.Cu") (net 6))
 (segment (start 86.875 38.125) (end 84.15 38.125) (width 0.25) (layer "F.Cu") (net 6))
 (segment (start 94.15 33.925) (end 102.57604 33.925) (width 0.25) (layer "F.Cu") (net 6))
 (segment (start 86.425 48.95) (end 86.425 49.825) (width 0.25) (layer "F.Cu") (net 6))
 (segment (start 85.75 48.275) (end 86.425 48.95) (width 0.25) (layer "F.Cu") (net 6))
 (segment (start 84.03498 38.24002) (end 84.03498 47.721618) (width 0.25) (layer "F.Cu") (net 6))
 (segment (start 101.207 51.1) (end 101.99727 51.89027) (width 0.25) (layer "F.Cu") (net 6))
 (segment (start 103.15 49.075) (end 103 48.925) (width 0.25) (layer "F.Cu") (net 6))
 (segment (start 105.299022 49.075) (end 105.05 49.075) (width 0.25) (layer "F.Cu") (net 6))
 (segment (start 93.55 44.25) (end 94.450489 44.25) (width 0.25) (layer "F.Cu") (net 6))
 (segment (start 86.425 49.825) (end 86.04573 49.44573) (width 0.25) (layer "F.Cu") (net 6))
 (segment (start 109.208 45.565) (end 109.204 45.569) (width 0.25) (layer "F.Cu") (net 6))
 (segment (start 91.475 48.6) (end 91.475 53.475) (width 0.25) (layer "F.Cu") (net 6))
 (segment (start 101.303 53.597) (end 101.303 52.606) (width 0.25) (layer "F.Cu") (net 6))
 (segment (start 109.208 41.0255) (end 109.208 45.565) (width 0.25) (layer "F.Cu") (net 6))
 (segment (start 110.356 45.569) (end 110.375 45.55) (width 0.25) (layer "F.Cu") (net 6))
 (segment (start 109.069 50.928) (end 107.403 50.928) (width 0.25) (layer "F.Cu") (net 6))
 (segment (start 93.35 45.5) (end 93.35 44.45) (width 0.25) (layer "F.Cu") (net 6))
 (segment (start 102.57604 33.925) (end 103.6 34.94896) (width 0.25) (layer "F.Cu") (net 6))
 (segment (start 109.204 45.569) (end 110.356 45.569) (width 0.25) (layer "F.Cu") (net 6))
 (segment (start 101.3 53.6) (end 101.303 53.597) (width 0.25) (layer "F.Cu") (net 6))
 (segment (start 91.6 53.6) (end 101.3 53.6) (width 0.25) (layer "F.Cu") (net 6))
 (segment (start 108.10673 51.89027) (end 109.069 50.928) (width 0.25) (layer "F.Cu") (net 6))
 (segment (start 98.682 48.575) (end 101.207 51.1) (width 0.25) (layer "F.Cu") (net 6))
 (segment (start 94.95 46.55) (end 96.975 48.575) (width 0.25) (layer "F.Cu") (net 6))
 (segment (start 93.35 44.45) (end 93.55 44.25) (width 0.25) (layer "F.Cu") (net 6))
 (segment (start 101.207 52.51) (end 101.303 52.606) (width 0.25) (layer "F.Cu") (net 6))
 (segment (start 97.525 48.575) (end 98.682 48.575) (width 0.25) (layer "F.Cu") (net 6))
 (segment (start 107.403 50.928) (end 107.25 50.775) (width 0.25) (layer "F.Cu") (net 6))
 (segment (start 91.75 45.5) (end 91.75 47) (width 0.25) (layer "F.Cu") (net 12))
 (segment (start 93.325 49.657) (end 94.868 51.2) (width 0.25) (layer "F.Cu") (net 12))
 (segment (start 93.325 48.575) (end 93.325 49.657) (width 0.25) (layer "F.Cu") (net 12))
 (segment (start 91.75 47) (end 93.325 48.575) (width 0.25) (layer "F.Cu") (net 12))
 (segment (start 93.325 48.575) (end 93.325 48.25) (width 0.25) (layer "F.Cu") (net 12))
 (segment (start 102.467859 45.582141) (end 102.5 45.55) (width 0.25) (layer "F.Cu") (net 17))
 (segment (start 99.975 41.85) (end 99.975 45.05048) (width 0.25) (layer "F.Cu") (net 17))
 (segment (start 101.236198 45.05048) (end 101.767859 45.582141) (width 0.25) (layer "F.Cu") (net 17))
 (segment (start 99.775 41.65) (end 99.975 41.85) (width 0.25) (layer "F.Cu") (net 17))
 (segment (start 101.767859 45.582141) (end 102.467859 45.582141) (width 0.25) (layer "F.Cu") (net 17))
 (segment (start 99.975 45.05048) (end 101.236198 45.05048) (width 0.25) (layer "F.Cu") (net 17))
 (segment (start 98.8 41.65) (end 99.775 41.65) (width 0.25) (layer "F.Cu") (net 17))
 (segment (start 102.475 44.025) (end 102.5 44) (width 0.25) (layer "F.Cu") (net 18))
 (segment (start 100.425 44.025) (end 102.475 44.025) (width 0.25) (layer "F.Cu") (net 18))
 (segment (start 100.425 41.275) (end 100.425 44.025) (width 0.25) (layer "F.Cu") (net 18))
 (segment (start 98.8 40.85) (end 100 40.85) (width 0.25) (layer "F.Cu") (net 18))
 (segment (start 100 40.85) (end 100.425 41.275) (width 0.25) (layer "F.Cu") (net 18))
 (segment (start 100.87452 42.525) (end 102.475 42.525) (width 0.25) (layer "F.Cu") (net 1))
 (segment (start 100.87452 41.088802) (end 100.87452 42.525) (width 0.25) (layer "F.Cu") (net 1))
 (segment (start 98.8 40.05) (end 99.835718 40.05) (width 0.25) (layer "F.Cu") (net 1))
 (segment (start 102.475 42.525) (end 102.5 42.5) (width 0.25) (layer "F.Cu") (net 1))
 (segment (start 99.835718 40.05) (end 100.87452 41.088802) (width 0.25) (layer "F.Cu") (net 1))
 (segment (start 87.47604 39.125) (end 88.45 40.09896) (width 0.25) (layer "F.Cu") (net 9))
 (segment (start 89.375978 42.45) (end 90.3 42.45) (width 0.25) (layer "F.Cu") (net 9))
 (segment (start 88.45 40.09896) (end 88.45 41.524022) (width 0.25) (layer "F.Cu") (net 9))
 (segment (start 86.875 39.125) (end 87.47604 39.125) (width 0.25) (layer "F.Cu") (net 9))
 (segment (start 88.45 41.524022) (end 89.375978 42.45) (width 0.25) (layer "F.Cu") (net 9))
 (segment (start 88.00048 41.874502) (end 89.375978 43.25) (width 0.25) (layer "F.Cu") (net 10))
 (segment (start 86.875 40.125) (end 87.47604 40.125) (width 0.25) (layer "F.Cu") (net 10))
 (segment (start 89.375978 43.25) (end 90.3 43.25) (width 0.25) (layer "F.Cu") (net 10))
 (segment (start 88.00048 40.64944) (end 88.00048 41.874502) (width 0.25) (layer "F.Cu") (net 10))
 (segment (start 87.47604 40.125) (end 88.00048 40.64944) (width 0.25) (layer "F.Cu") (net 10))
 (segment (start 103.45 36.55) (end 100.75 39.25) (width 0.25) (layer "F.Cu") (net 19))
 (segment (start 100.625 39.25) (end 100.75 39.25) (width 0.25) (layer "F.Cu") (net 19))
 (segment (start 103.6 36.55) (end 103.45 36.55) (width 0.25) (layer "F.Cu") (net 19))
 (segment (start 98.8 39.25) (end 100.625 39.25) (width 0.25) (layer "F.Cu") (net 19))
 (segment (start 100.75 39.25) (end 102.5 41) (width 0.25) (layer "F.Cu") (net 19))
 (segment (start 107.25 49.075) (end 108.89 49.075) (width 0.25) (layer "F.Cu") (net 5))
 (segment (start 106.85 47.45) (end 100.075 47.45) (width 0.25) (layer "F.Cu") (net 5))
 (segment (start 100.075 47.45) (end 98.125 45.5) (width 0.25) (layer "F.Cu") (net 5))
 (segment (start 107.25 49.075) (end 107.25 47.85) (width 0.25) (layer "F.Cu") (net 5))
 (segment (start 108.89 49.075) (end 109.069 48.896) (width 0.25) (layer "F.Cu") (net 5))
 (segment (start 107.25 47.85) (end 106.85 47.45) (width 0.25) (layer "F.Cu") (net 5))
 (segment (start 98.125 45.5) (end 97.35 45.5) (width 0.25) (layer "F.Cu") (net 5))
 (segment (start 99.29348 47.25048) (end 103 50.957) (width 0.25) (layer "F.Cu") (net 7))
 (segment (start 105.05 50.775) (end 103.182 50.775) (width 0.25) (layer "F.Cu") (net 7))
 (segment (start 96.55 45.5) (end 96.55 46.55) (width 0.25) (layer "F.Cu") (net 7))
 (segment (start 103.182 50.775) (end 103 50.957) (width 0.25) (layer "F.Cu") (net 7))
 (segment (start 96.55 46.55) (end 97.25048 47.25048) (width 0.25) (layer "F.Cu") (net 7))
 (segment (start 97.25048 47.25048) (end 99.29348 47.25048) (width 0.25) (layer "F.Cu") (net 7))
 (segment (start 84.947 47.269) (end 84.947 42.99303) (width 0.25) (layer "F.Cu") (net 3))
 (segment (start 86.93497 41.125) (end 86.875 41.125) (width 0.25) (layer "F.Cu") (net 3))
 (segment (start 84.947 42.99303) (end 86.81503 41.125) (width 0.25) (layer "F.Cu") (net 3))
 (segment (start 86.81503 41.125) (end 86.875 41.125) (width 0.25) (layer "F.Cu") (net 3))
 (segment (start 104.532 45.55) (end 107.153 45.55) (width 0.25) (layer "F.Cu") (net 32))
 (segment (start 107.153 45.55) (end 107.172 45.569) (width 0.25) (layer "F.Cu") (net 32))
 (segment (start 104.532 44) (end 107.15 44) (width 0.25) (layer "F.Cu") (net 31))
 (segment (start 107.15 44) (end 107.175 44.025) (width 0.25) (layer "F.Cu") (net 31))
 (segment (start 107.1405 42.5) (end 107.172 42.5315) (width 0.25) (layer "F.Cu") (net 2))
 (segment (start 104.532 42.5) (end 107.1405 42.5) (width 0.25) (layer "F.Cu") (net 2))
 (segment (start 104.532 41) (end 104.5575 41.0255) (width 0.25) (layer "F.Cu") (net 33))
 (segment (start 104.5575 41.0255) (end 107.176 41.0255) (width 0.25) (layer "F.Cu") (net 33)))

